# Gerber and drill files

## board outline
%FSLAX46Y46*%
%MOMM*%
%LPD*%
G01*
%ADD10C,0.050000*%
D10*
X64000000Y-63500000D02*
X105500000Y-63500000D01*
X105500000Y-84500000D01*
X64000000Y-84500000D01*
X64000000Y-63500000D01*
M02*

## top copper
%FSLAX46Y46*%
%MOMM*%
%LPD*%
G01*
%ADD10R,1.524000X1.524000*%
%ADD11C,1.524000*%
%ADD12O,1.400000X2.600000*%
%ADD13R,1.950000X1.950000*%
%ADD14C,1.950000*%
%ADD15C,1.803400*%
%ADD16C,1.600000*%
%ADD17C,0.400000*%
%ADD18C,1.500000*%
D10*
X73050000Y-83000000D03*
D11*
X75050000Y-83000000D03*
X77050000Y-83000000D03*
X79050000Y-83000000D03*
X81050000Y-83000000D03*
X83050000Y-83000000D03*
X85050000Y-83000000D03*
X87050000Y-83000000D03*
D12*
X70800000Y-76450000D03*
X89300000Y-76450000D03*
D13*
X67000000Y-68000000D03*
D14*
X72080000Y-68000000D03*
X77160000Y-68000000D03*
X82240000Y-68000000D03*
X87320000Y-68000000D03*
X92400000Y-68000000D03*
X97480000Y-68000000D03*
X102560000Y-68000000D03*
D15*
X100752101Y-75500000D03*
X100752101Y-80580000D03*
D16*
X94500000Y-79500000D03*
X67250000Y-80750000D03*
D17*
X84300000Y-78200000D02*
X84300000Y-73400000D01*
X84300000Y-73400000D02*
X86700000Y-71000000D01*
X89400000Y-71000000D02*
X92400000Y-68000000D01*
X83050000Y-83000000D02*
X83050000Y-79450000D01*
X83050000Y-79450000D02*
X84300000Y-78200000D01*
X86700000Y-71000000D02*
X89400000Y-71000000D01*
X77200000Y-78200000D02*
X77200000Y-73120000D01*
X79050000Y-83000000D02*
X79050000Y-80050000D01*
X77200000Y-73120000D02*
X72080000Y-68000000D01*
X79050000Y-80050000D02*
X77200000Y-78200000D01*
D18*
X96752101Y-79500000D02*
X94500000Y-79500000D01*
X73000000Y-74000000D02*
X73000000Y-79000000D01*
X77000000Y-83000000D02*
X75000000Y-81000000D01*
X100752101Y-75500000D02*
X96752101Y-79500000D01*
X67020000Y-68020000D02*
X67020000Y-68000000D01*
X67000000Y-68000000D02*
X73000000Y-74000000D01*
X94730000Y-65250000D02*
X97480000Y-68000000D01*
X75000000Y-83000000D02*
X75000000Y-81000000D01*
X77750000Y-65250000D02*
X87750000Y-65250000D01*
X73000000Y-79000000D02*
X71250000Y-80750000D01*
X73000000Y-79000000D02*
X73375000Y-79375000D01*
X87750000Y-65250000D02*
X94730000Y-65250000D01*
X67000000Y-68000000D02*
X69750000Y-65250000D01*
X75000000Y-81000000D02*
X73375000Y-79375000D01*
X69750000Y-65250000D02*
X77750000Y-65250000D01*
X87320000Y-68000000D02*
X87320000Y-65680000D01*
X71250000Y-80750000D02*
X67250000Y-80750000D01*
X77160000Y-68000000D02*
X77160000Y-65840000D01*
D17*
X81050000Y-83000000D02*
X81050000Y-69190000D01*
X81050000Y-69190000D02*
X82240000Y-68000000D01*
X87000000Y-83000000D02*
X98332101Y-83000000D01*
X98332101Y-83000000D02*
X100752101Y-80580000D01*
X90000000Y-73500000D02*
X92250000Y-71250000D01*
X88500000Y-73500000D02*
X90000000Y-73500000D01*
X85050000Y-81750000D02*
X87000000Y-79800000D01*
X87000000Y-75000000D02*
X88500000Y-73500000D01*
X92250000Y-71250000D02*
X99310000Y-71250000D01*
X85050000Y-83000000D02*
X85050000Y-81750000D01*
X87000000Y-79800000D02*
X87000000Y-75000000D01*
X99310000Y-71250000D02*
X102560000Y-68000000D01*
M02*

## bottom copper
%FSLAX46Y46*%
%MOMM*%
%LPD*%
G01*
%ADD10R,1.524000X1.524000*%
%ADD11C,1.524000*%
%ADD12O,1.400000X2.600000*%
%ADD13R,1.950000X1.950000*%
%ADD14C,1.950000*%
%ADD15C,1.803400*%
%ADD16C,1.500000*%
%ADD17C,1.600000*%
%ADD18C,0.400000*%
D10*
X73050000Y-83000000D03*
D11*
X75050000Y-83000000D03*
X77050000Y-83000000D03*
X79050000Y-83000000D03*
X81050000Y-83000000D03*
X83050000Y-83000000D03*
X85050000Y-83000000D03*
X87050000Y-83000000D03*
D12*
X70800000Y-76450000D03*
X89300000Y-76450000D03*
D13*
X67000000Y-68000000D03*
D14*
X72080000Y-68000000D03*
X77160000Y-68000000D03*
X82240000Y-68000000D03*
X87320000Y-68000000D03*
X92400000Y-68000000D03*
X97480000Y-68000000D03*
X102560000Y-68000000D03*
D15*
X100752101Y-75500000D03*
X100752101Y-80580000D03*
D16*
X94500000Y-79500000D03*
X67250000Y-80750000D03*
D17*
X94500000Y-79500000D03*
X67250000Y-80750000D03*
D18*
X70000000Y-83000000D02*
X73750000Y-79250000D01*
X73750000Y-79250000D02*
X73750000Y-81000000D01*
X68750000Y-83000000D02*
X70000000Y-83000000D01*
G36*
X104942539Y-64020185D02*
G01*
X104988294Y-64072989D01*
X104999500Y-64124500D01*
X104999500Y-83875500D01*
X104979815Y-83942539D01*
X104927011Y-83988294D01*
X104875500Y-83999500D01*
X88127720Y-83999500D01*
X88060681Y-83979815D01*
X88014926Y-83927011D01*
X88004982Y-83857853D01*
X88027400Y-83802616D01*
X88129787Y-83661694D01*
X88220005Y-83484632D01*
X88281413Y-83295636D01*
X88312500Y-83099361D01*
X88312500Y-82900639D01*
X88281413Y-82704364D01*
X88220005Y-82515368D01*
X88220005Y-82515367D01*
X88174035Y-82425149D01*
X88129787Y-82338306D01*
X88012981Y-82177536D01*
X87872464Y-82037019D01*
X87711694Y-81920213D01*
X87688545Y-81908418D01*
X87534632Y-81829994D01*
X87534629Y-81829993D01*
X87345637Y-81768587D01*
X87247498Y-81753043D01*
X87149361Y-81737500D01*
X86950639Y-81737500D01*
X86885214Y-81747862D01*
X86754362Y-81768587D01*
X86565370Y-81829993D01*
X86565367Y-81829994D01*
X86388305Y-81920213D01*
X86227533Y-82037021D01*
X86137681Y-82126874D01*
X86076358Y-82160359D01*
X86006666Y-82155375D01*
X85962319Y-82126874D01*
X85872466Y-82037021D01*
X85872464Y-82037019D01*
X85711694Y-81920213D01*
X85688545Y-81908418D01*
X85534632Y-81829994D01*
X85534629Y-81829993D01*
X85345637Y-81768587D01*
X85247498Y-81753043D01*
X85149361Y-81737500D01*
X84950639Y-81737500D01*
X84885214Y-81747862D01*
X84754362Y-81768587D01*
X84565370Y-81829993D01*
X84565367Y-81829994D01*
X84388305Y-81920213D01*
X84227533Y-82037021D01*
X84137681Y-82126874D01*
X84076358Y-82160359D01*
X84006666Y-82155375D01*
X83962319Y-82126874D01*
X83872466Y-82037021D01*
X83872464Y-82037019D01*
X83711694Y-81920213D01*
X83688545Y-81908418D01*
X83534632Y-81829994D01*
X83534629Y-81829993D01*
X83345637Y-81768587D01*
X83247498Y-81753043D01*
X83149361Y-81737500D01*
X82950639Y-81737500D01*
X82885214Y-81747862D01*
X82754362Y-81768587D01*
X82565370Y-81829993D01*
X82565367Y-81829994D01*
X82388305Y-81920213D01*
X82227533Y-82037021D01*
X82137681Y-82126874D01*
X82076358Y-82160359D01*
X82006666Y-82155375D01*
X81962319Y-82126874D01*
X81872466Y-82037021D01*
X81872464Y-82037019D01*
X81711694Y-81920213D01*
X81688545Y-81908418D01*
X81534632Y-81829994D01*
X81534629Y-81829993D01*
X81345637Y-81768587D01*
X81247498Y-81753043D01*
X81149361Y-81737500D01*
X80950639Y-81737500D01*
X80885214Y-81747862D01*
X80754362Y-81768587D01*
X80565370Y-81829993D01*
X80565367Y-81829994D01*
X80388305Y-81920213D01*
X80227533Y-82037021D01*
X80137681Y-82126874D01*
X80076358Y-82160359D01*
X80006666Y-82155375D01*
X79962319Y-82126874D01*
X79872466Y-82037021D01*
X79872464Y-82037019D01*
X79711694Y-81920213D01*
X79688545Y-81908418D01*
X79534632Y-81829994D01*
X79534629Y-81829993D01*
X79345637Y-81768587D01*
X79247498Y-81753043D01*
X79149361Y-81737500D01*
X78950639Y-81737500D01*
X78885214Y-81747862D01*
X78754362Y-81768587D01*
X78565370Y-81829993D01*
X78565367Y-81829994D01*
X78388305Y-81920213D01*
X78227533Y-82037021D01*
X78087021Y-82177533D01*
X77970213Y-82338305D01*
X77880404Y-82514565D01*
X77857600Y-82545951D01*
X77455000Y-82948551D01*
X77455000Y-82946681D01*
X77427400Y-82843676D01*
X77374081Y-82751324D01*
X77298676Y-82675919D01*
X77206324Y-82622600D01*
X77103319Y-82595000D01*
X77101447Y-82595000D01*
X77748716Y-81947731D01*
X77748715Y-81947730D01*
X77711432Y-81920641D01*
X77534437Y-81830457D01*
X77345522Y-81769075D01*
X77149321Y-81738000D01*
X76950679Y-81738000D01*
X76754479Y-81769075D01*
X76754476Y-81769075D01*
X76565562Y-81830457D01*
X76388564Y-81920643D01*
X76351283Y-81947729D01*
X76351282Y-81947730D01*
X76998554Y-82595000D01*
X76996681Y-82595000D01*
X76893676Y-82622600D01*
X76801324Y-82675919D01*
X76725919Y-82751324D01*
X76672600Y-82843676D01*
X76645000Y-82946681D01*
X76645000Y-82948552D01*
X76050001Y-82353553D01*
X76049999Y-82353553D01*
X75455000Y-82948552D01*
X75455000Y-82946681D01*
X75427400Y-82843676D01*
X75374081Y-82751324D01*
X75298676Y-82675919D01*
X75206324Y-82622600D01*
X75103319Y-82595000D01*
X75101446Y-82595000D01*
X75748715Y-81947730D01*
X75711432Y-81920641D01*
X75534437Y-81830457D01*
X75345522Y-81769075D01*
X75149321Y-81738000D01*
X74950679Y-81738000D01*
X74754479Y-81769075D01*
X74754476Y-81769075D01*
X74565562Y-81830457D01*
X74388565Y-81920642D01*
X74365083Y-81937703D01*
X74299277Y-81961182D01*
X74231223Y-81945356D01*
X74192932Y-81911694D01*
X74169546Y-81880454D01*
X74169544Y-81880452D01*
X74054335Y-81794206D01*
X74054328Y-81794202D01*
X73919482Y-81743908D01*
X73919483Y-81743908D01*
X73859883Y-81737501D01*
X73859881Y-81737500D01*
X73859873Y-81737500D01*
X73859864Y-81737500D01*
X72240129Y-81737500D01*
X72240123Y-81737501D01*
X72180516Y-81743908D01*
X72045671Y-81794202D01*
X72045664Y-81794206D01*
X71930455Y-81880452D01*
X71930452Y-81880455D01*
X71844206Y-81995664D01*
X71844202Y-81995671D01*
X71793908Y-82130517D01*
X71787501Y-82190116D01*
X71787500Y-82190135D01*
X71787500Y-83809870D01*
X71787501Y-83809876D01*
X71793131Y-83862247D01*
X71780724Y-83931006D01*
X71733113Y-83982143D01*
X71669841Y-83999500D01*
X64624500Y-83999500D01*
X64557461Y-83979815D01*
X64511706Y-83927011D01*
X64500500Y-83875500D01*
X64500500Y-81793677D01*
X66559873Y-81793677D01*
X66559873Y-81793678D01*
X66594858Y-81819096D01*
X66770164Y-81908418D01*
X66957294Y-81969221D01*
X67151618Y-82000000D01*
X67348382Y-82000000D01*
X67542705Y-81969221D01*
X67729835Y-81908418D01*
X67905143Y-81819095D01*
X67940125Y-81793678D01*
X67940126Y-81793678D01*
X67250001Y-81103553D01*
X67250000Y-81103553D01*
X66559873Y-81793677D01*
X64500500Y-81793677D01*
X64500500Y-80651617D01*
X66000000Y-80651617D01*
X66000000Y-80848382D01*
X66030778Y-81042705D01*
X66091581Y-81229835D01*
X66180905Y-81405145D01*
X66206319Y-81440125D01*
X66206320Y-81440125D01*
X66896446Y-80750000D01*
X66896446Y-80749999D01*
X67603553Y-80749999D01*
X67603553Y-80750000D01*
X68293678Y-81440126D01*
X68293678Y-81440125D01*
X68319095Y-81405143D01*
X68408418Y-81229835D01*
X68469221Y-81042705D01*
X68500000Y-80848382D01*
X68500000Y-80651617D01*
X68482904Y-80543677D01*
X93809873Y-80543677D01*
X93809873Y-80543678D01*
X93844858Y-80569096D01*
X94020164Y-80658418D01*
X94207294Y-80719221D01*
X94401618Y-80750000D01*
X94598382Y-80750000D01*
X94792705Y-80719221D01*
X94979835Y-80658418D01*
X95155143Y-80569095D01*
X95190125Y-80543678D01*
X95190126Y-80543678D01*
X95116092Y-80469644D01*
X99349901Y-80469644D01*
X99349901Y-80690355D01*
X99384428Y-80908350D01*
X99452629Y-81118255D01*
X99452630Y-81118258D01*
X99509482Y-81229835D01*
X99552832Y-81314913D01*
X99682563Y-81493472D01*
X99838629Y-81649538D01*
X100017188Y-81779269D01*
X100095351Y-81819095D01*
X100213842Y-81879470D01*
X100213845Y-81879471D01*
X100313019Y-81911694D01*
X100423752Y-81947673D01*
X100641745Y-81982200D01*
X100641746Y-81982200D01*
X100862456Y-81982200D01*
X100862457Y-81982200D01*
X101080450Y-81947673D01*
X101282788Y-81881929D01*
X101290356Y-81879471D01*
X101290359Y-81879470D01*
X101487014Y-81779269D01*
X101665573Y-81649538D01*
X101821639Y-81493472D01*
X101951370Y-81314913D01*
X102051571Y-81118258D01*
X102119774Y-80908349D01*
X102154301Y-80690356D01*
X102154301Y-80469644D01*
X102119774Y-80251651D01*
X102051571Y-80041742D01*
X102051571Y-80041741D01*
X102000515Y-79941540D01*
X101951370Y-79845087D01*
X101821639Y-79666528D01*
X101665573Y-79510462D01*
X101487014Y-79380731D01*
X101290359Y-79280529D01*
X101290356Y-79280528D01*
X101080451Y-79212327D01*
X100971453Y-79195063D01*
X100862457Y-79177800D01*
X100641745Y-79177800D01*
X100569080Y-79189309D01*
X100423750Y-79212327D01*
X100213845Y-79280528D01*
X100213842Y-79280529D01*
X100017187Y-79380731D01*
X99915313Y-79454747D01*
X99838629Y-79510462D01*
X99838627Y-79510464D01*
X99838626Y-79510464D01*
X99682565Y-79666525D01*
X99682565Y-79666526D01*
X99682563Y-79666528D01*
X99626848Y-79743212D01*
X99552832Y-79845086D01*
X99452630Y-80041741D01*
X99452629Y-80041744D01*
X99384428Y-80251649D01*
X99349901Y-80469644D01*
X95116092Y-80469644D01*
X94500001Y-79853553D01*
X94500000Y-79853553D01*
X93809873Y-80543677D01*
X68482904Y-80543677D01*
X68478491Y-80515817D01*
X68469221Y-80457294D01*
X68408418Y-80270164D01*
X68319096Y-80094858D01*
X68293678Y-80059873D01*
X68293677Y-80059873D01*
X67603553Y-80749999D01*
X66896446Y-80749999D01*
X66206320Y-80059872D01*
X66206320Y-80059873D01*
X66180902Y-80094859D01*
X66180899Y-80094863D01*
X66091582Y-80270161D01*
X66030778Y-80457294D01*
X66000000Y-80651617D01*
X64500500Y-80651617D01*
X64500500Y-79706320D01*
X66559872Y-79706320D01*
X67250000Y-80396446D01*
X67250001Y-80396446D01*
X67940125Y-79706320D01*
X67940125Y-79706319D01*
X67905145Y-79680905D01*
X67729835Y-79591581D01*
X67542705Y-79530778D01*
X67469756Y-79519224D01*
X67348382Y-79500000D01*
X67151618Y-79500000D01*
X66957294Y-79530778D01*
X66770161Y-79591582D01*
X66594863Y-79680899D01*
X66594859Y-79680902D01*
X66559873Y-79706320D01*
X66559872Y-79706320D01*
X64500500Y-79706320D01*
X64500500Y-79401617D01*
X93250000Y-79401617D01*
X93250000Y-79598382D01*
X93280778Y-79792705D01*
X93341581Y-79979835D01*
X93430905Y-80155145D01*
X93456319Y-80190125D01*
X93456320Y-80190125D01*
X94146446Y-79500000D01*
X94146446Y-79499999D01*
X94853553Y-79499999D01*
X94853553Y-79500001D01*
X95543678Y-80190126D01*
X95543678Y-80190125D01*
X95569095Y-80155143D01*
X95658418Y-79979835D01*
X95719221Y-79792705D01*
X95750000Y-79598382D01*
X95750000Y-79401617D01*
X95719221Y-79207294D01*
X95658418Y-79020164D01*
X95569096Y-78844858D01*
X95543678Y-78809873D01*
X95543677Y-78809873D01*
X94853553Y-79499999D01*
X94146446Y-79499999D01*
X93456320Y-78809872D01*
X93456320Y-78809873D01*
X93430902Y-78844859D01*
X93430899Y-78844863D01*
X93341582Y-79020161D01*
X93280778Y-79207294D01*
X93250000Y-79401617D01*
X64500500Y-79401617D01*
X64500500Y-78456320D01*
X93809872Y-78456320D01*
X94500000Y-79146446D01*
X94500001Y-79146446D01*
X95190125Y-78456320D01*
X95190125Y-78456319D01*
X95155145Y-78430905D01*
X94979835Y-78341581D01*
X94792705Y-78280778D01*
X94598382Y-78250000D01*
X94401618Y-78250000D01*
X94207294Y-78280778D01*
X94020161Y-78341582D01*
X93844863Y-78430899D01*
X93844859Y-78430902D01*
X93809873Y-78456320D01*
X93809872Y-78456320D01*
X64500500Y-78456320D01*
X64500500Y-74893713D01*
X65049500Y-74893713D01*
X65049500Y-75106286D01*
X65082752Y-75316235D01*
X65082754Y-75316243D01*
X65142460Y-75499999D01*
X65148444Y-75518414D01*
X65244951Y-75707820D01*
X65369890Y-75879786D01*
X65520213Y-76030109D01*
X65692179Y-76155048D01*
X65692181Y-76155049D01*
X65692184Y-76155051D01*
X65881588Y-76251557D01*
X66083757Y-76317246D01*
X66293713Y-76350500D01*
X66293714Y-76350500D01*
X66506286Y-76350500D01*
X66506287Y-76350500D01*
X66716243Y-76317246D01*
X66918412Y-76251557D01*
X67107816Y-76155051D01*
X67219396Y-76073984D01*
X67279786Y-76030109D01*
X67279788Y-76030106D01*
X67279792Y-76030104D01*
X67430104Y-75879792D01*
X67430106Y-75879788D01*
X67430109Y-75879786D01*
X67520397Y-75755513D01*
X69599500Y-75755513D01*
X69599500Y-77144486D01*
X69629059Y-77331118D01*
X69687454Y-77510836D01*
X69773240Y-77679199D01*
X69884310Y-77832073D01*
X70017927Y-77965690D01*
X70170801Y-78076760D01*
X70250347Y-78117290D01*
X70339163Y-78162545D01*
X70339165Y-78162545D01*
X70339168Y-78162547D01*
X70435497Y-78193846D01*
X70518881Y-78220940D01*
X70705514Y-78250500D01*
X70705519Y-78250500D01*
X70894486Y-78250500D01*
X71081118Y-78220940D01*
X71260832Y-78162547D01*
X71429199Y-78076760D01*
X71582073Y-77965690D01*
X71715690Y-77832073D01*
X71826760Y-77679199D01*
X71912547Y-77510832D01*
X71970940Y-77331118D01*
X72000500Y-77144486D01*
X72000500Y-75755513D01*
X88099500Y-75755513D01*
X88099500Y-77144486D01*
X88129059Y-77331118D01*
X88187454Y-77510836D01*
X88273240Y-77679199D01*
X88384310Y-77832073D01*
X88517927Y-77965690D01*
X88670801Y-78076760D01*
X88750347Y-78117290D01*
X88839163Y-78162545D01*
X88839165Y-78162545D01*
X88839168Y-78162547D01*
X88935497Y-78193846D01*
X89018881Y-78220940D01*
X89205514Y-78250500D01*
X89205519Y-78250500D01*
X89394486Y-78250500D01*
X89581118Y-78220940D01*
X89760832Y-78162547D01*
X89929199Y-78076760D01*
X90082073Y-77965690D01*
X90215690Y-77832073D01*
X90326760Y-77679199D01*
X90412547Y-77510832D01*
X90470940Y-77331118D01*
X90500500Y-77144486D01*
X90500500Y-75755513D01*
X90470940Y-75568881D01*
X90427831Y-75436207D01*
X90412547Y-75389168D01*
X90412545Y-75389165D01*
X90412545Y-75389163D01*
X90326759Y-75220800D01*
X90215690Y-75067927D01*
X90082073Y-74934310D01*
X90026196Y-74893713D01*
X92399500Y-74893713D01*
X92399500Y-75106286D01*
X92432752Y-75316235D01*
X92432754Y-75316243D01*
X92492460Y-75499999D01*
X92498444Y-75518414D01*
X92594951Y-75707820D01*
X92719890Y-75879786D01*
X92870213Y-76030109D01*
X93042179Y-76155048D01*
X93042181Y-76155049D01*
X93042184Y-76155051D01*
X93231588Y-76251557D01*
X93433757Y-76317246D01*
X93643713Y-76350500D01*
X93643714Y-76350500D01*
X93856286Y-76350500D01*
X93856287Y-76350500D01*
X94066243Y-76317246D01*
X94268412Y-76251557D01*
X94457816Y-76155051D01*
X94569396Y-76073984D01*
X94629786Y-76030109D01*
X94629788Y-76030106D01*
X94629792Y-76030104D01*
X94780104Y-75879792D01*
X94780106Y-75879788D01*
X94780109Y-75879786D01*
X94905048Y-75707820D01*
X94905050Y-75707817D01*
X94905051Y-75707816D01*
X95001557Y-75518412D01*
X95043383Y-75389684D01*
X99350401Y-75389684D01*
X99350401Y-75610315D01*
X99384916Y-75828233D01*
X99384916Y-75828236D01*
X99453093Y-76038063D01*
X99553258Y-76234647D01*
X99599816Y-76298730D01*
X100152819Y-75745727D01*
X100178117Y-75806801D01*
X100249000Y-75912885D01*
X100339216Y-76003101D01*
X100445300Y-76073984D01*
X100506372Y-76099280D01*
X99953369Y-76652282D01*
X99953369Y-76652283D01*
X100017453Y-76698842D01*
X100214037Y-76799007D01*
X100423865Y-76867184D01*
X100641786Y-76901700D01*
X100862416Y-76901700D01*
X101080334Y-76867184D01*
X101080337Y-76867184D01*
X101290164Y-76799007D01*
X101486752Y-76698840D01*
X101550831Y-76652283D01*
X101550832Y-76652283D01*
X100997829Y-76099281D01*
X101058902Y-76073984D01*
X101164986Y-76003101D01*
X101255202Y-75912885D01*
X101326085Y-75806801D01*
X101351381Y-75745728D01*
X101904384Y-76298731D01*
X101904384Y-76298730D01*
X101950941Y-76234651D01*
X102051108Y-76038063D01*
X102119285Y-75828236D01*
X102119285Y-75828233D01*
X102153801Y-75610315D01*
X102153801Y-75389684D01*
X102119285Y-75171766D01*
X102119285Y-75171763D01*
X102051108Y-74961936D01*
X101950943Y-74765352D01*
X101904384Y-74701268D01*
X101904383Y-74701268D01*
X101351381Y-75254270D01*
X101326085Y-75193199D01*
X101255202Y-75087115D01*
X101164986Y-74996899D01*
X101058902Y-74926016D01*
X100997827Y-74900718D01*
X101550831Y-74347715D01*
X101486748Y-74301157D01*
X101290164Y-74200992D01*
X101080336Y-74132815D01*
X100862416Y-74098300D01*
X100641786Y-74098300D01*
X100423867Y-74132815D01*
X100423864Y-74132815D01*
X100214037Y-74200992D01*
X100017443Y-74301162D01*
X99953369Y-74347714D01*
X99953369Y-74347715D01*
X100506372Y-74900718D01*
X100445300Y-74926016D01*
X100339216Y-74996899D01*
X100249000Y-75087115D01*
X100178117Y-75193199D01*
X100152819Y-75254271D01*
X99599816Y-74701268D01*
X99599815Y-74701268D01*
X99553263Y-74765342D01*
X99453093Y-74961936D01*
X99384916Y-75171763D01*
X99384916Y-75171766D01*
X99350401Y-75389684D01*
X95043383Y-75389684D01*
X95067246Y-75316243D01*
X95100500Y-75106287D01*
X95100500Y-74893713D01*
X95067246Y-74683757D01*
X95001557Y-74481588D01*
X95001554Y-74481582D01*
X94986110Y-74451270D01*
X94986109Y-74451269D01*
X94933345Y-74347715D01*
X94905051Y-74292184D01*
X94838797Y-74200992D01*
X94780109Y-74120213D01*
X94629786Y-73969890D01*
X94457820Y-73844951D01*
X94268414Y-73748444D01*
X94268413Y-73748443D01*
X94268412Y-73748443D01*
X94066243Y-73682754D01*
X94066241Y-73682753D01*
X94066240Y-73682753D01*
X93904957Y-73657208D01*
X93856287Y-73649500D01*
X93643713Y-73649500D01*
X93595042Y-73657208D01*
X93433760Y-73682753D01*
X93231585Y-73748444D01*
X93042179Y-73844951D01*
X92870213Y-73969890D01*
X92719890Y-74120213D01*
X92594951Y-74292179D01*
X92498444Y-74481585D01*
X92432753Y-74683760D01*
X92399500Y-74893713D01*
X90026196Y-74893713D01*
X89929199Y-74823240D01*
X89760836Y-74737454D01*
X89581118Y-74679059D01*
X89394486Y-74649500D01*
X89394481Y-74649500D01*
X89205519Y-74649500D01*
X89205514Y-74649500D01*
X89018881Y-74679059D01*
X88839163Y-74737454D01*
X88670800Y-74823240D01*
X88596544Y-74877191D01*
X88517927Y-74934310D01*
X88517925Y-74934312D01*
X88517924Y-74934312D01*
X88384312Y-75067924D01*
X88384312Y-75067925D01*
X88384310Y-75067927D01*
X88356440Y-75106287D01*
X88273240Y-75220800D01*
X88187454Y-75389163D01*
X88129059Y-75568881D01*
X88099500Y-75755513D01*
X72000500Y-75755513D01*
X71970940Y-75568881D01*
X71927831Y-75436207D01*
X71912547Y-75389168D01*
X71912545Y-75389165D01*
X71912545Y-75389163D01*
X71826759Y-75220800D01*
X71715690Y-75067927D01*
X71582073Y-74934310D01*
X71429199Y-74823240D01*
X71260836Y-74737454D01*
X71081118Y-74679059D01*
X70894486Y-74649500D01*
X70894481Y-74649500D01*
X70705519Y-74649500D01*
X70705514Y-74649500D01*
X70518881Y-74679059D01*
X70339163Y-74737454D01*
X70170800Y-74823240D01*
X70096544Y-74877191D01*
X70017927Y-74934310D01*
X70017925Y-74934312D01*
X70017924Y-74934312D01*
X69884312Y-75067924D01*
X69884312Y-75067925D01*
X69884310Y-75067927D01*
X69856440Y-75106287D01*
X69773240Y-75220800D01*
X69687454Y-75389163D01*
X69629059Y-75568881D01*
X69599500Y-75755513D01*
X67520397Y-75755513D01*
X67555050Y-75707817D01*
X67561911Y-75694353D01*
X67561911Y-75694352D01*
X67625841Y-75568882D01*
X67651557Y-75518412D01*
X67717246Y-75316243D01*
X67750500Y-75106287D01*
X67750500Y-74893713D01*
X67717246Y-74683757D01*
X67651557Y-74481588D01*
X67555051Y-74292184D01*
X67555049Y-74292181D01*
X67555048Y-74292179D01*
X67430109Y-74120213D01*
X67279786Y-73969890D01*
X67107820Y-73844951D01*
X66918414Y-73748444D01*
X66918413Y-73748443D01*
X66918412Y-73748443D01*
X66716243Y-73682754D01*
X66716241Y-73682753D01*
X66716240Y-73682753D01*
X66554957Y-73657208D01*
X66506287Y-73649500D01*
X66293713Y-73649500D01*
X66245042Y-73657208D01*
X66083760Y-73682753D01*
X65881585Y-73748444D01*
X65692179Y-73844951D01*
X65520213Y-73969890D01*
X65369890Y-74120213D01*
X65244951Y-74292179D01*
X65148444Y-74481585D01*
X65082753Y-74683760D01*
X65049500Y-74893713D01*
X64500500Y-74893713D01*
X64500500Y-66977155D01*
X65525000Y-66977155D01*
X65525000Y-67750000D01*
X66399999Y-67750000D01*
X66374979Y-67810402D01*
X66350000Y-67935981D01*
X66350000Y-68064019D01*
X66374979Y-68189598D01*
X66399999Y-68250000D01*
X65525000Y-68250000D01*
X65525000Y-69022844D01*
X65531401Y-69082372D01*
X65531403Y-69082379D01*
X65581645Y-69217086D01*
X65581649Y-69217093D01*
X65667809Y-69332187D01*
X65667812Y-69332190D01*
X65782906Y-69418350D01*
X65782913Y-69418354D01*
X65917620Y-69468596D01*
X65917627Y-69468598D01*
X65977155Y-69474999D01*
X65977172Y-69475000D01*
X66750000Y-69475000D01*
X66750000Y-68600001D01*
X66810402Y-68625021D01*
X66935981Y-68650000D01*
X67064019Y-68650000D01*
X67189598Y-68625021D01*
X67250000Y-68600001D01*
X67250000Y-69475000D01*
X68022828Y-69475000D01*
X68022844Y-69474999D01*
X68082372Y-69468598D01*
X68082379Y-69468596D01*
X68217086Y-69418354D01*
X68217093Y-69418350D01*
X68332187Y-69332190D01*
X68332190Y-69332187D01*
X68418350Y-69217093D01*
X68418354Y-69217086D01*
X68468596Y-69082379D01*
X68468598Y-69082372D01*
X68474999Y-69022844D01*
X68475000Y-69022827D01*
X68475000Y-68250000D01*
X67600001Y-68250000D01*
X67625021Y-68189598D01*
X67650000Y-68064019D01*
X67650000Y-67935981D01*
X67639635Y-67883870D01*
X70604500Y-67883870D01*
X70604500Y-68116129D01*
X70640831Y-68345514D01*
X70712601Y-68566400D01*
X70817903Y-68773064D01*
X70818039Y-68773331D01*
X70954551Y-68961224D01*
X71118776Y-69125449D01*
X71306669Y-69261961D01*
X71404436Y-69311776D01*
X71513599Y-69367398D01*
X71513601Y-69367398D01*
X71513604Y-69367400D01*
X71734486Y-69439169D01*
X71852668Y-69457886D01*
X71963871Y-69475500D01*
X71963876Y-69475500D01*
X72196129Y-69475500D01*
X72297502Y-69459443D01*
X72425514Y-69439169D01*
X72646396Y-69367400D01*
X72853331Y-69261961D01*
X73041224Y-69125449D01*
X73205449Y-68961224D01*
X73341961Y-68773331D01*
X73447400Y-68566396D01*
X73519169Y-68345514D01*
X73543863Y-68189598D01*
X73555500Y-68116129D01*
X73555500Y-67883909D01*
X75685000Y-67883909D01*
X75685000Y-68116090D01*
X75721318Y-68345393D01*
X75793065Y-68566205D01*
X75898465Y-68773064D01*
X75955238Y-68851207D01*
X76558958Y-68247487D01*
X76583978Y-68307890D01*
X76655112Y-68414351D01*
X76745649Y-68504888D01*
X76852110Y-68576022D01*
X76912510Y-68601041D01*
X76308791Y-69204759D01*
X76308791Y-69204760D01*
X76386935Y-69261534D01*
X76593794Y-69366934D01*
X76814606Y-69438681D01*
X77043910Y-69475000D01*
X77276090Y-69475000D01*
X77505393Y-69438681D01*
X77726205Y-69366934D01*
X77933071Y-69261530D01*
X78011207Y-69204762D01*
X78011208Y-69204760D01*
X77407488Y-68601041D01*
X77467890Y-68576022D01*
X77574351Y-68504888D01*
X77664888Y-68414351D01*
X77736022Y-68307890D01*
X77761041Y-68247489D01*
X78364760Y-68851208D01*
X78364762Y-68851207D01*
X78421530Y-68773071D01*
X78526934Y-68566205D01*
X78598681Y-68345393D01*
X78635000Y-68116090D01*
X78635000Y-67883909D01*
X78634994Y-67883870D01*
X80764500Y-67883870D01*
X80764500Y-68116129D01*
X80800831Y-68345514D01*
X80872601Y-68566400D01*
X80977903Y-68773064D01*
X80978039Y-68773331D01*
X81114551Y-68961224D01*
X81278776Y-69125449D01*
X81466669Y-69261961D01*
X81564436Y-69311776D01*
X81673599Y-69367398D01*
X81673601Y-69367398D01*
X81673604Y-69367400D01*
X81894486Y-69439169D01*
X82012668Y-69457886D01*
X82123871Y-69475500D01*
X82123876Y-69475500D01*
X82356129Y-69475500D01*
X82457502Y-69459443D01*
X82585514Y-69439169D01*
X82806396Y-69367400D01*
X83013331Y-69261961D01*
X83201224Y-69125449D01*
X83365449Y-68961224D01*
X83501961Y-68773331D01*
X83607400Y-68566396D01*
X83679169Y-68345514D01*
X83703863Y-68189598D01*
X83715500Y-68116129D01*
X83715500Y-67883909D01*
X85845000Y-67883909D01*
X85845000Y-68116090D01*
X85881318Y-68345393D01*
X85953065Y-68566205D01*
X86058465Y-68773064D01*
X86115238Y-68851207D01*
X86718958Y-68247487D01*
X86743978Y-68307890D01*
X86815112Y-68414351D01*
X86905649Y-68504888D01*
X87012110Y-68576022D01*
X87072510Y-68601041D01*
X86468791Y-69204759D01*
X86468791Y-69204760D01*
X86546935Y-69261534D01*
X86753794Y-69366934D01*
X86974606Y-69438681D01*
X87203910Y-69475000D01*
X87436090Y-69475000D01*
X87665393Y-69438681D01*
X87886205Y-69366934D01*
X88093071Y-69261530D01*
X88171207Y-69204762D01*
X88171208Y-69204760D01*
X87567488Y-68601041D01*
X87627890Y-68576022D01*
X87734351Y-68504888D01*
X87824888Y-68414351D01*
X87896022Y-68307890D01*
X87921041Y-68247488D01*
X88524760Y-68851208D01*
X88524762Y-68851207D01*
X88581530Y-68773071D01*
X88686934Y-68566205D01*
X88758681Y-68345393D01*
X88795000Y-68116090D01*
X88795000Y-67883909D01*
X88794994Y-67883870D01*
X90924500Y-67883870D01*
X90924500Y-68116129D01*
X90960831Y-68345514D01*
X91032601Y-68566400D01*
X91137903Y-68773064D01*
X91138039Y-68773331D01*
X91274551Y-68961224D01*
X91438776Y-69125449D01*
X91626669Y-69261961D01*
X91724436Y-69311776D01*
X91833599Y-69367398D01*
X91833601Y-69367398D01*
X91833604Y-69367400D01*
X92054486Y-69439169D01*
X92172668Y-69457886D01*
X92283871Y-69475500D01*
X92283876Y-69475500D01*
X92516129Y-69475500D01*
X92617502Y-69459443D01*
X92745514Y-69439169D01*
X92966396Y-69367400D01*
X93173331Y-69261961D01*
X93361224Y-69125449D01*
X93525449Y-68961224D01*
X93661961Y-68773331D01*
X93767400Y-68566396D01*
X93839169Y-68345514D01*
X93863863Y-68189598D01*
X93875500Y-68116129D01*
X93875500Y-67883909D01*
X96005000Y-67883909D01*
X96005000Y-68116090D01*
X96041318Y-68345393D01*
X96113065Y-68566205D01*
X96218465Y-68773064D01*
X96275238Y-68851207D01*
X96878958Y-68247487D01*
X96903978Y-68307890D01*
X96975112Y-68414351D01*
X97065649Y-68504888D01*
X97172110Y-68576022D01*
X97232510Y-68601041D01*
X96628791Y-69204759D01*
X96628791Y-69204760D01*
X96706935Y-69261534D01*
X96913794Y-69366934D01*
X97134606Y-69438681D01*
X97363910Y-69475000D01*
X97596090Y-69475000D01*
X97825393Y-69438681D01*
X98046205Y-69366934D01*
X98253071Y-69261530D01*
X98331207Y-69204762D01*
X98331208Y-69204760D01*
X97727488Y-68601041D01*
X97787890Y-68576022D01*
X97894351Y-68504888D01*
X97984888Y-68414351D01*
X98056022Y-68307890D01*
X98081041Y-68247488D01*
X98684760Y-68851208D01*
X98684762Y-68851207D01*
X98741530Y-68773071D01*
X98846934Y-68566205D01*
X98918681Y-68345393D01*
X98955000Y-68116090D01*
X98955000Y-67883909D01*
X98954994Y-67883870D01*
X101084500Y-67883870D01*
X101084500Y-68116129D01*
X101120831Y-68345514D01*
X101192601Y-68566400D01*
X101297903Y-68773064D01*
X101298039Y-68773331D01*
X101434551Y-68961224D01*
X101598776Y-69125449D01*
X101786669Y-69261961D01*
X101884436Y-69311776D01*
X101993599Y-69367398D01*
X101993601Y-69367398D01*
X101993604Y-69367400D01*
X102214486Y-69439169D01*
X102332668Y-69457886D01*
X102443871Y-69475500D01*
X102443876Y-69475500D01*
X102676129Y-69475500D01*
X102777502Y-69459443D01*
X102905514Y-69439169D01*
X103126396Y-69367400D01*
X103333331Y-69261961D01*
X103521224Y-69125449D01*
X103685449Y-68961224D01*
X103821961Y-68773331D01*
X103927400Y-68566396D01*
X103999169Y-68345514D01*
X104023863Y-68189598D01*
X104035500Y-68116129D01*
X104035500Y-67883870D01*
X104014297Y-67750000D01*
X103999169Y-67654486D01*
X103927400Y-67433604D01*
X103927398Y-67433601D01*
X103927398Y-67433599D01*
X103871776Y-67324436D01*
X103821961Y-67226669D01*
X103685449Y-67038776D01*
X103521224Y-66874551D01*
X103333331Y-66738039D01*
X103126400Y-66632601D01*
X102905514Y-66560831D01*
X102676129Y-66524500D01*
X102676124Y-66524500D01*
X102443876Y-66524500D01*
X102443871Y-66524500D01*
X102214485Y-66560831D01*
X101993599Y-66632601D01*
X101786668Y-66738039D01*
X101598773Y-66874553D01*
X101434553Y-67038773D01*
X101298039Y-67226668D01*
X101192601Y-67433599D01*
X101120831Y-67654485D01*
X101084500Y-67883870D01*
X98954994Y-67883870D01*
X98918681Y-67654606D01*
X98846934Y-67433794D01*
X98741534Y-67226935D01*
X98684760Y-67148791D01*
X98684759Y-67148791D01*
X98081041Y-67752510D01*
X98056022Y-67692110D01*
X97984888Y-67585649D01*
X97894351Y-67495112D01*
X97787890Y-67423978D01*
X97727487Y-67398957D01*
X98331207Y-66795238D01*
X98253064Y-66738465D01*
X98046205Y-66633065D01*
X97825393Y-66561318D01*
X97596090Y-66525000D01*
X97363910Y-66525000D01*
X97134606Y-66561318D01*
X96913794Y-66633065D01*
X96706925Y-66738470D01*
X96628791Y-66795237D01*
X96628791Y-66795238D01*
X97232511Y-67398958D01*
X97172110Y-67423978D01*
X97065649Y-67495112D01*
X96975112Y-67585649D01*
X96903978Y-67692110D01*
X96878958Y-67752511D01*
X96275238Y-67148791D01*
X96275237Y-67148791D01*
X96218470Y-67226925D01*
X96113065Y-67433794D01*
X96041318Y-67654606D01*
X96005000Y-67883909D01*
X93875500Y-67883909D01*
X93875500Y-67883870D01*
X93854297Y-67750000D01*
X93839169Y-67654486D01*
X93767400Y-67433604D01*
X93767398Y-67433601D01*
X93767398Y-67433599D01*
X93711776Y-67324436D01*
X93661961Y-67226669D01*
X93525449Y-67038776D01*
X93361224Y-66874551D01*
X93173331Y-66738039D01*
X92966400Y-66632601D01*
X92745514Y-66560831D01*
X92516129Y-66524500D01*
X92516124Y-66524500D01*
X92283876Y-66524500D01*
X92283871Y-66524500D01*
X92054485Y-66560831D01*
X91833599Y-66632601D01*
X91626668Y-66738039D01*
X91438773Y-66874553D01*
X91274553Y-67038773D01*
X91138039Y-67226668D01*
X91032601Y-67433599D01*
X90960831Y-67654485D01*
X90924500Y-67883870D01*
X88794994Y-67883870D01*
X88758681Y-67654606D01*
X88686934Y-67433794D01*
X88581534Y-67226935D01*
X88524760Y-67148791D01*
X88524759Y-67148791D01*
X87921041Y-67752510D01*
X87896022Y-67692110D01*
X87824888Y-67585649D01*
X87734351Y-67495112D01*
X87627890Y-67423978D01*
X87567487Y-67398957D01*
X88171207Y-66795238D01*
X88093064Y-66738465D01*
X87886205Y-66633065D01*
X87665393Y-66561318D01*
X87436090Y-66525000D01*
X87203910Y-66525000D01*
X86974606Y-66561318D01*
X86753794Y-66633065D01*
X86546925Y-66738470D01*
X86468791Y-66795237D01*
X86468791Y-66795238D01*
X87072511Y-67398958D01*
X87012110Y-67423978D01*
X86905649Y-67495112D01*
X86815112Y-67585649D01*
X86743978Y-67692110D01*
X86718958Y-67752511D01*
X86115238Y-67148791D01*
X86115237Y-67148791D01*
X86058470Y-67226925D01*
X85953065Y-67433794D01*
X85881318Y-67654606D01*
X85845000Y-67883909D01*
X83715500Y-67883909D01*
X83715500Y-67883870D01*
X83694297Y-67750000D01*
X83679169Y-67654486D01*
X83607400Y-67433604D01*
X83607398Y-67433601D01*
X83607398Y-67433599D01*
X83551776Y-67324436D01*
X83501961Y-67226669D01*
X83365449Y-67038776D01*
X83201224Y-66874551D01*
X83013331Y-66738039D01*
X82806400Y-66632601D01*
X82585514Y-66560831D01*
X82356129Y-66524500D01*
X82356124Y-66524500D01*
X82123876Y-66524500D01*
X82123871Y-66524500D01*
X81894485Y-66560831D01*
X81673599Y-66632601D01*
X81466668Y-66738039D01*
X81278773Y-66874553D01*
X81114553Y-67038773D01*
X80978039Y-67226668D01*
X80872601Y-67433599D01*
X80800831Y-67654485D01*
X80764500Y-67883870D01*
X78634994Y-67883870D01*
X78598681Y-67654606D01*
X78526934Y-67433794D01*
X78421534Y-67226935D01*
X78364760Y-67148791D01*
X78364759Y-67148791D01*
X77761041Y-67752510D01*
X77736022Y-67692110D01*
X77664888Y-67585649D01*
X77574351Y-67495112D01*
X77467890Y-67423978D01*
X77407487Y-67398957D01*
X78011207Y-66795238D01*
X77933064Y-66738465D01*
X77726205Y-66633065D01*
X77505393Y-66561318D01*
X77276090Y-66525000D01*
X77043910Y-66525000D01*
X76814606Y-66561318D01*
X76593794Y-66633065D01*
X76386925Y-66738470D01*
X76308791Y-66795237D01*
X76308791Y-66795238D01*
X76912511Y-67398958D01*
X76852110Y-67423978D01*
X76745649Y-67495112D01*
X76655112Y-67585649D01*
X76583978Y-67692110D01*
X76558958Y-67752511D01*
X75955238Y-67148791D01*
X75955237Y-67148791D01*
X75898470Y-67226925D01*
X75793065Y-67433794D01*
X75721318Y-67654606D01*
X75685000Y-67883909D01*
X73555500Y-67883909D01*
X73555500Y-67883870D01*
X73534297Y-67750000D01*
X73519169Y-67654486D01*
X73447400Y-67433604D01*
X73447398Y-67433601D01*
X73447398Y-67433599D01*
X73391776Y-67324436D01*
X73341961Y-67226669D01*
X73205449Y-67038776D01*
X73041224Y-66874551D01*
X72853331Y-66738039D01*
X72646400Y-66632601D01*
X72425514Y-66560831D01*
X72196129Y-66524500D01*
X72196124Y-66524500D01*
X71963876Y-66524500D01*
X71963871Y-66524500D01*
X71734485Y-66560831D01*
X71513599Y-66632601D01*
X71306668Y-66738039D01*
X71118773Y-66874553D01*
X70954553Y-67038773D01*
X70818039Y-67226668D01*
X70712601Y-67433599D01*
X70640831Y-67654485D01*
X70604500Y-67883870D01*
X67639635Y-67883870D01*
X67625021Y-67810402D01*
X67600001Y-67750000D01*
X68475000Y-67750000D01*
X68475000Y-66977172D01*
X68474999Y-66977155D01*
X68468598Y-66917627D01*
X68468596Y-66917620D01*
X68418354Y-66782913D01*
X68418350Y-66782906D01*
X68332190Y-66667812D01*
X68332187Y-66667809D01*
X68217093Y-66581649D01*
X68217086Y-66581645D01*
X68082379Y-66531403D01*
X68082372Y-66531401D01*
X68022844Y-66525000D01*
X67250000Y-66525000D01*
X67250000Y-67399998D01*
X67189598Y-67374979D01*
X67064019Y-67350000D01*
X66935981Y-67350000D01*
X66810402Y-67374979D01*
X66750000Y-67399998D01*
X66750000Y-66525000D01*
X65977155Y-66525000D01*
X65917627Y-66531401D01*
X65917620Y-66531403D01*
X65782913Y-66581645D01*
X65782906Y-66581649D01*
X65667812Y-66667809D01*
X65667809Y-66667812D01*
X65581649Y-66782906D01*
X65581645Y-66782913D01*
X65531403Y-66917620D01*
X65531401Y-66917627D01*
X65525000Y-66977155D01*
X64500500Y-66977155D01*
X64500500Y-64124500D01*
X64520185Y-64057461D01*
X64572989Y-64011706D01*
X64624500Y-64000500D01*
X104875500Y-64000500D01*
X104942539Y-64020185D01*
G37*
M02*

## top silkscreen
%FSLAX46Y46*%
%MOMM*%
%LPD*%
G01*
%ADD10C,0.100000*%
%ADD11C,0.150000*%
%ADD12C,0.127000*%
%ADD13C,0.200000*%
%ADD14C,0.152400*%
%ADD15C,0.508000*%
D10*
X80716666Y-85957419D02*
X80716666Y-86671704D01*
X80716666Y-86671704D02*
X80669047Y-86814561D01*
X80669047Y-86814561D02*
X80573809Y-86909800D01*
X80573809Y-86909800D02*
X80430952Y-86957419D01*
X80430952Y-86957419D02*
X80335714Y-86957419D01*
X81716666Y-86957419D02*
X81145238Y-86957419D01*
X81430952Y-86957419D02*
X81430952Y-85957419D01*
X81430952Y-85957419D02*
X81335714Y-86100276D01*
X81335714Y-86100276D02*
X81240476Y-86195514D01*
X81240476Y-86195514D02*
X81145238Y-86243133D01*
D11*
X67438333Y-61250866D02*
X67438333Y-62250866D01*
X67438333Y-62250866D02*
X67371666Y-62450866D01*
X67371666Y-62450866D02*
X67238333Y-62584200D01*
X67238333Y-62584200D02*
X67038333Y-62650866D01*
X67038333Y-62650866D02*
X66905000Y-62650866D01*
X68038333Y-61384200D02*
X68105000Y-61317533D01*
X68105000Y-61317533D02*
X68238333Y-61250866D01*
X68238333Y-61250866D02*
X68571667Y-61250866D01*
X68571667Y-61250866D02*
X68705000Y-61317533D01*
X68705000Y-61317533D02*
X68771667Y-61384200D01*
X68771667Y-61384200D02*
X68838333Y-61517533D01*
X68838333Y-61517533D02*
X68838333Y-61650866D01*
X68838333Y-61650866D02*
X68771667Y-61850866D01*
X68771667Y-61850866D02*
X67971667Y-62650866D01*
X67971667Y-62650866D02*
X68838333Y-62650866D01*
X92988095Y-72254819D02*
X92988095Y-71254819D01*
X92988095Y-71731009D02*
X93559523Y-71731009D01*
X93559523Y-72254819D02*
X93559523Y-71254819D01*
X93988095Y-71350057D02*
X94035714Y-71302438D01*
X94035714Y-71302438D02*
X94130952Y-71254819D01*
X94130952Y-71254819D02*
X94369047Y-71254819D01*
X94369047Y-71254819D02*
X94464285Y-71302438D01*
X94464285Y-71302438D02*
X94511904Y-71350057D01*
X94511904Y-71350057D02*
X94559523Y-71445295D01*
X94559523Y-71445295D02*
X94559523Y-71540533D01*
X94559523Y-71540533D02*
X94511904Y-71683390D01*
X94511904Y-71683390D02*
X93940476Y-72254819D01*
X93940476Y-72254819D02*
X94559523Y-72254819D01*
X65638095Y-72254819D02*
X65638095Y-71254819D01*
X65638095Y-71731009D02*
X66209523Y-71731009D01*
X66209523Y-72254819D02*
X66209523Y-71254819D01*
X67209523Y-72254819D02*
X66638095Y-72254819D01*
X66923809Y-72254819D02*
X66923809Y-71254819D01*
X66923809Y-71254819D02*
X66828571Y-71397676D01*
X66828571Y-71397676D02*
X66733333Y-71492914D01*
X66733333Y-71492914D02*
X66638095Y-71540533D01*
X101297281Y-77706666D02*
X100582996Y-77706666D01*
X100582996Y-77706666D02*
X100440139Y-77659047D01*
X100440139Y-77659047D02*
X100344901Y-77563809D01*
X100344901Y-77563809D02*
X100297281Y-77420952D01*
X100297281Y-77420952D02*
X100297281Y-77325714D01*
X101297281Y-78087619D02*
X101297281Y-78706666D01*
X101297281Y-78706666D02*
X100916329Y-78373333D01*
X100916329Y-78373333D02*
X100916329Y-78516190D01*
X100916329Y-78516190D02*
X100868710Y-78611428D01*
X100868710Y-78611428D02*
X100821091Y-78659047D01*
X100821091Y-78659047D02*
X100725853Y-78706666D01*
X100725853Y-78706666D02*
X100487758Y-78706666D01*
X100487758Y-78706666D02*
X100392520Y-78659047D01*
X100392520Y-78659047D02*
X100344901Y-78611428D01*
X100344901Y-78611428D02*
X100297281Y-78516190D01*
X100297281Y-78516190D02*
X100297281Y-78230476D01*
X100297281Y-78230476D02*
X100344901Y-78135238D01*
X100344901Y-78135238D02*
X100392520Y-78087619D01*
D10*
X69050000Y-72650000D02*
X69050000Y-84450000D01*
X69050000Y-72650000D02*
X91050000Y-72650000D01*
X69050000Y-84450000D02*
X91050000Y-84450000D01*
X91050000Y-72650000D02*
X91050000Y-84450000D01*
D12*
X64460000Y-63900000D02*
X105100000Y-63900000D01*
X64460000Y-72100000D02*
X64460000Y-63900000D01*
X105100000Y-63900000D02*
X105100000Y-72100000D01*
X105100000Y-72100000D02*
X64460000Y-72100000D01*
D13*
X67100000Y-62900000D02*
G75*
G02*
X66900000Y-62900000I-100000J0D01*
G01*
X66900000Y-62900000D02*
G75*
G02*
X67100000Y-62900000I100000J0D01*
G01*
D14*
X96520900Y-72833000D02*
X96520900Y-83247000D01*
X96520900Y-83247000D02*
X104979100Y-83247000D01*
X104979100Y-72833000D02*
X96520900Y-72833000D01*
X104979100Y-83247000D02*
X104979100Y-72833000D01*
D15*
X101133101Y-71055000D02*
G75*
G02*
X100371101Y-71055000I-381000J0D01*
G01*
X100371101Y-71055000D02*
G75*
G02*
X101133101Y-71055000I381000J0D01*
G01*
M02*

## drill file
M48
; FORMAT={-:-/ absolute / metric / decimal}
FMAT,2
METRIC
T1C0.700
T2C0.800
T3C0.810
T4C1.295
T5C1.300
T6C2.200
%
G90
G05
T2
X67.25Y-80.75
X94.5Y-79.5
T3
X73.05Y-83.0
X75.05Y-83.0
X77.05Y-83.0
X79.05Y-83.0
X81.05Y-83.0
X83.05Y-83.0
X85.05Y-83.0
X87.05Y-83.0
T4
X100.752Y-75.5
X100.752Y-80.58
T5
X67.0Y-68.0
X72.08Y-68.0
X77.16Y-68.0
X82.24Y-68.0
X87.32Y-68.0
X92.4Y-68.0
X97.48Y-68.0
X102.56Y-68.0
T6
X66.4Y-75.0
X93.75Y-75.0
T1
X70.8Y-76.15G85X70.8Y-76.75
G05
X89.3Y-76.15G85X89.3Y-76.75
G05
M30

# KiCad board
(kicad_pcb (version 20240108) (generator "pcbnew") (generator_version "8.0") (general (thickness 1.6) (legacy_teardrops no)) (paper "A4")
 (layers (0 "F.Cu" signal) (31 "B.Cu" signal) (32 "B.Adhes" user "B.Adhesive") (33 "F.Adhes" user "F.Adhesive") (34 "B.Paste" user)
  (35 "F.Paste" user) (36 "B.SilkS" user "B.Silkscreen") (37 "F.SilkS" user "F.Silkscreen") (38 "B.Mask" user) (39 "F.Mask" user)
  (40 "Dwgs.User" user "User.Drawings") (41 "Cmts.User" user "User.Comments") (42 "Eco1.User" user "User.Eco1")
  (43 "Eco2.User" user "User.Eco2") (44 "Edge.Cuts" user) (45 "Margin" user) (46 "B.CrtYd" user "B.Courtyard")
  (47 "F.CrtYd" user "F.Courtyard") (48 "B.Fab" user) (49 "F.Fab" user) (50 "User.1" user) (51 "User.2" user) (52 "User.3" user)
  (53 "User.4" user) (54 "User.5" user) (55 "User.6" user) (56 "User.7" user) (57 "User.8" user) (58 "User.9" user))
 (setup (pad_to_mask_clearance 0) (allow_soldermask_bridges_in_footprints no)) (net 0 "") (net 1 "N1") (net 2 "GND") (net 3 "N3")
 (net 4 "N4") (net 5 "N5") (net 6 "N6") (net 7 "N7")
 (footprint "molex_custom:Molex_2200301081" (layer "F.Cu") (at 81.05 87)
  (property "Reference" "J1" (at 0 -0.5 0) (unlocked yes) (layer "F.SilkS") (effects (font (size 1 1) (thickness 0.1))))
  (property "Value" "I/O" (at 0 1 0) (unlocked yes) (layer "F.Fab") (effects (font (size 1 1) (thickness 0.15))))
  (fp_line (start -12 -14.35) (end -12 -2.55) (stroke (width 0.1) (type default)) (layer "F.SilkS"))
  (fp_line (start -12 -14.35) (end 10 -14.35) (stroke (width 0.1) (type default)) (layer "F.SilkS"))
  (fp_line (start -12 -2.55) (end 10 -2.55) (stroke (width 0.1) (type default)) (layer "F.SilkS"))
  (fp_line (start 10 -14.35) (end 10 -2.55) (stroke (width 0.1) (type default)) (layer "F.SilkS"))
  (pad "1" thru_hole rect (at -8 -4 90) (size 1.524 1.524) (drill 0.81) (layers "*.Cu" "*.Mask") (remove_unused_layers no) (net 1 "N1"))
  (pad "2" thru_hole circle (at -6 -4 90) (size 1.524 1.524) (drill 0.81) (layers "*.Cu" "*.Mask") (remove_unused_layers no) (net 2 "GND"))
  (pad "3" thru_hole circle (at -4 -4 90) (size 1.524 1.524) (drill 0.81) (layers "*.Cu" "*.Mask") (remove_unused_layers no) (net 2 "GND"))
  (pad "4" thru_hole circle (at -2 -4 90) (size 1.524 1.524) (drill 0.81) (layers "*.Cu" "*.Mask") (remove_unused_layers no) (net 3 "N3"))
  (pad "5" thru_hole circle (at 0 -4 90) (size 1.524 1.524) (drill 0.81) (layers "*.Cu" "*.Mask") (remove_unused_layers no) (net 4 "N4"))
  (pad "6" thru_hole circle (at 2 -4 90) (size 1.524 1.524) (drill 0.81) (layers "*.Cu" "*.Mask") (remove_unused_layers no) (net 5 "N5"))
  (pad "7" thru_hole circle (at 4 -4 90) (size 1.524 1.524) (drill 0.81) (layers "*.Cu" "*.Mask") (remove_unused_layers no) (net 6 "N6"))
  (pad "8" thru_hole circle (at 6 -4 90) (size 1.524 1.524) (drill 0.81) (layers "*.Cu" "*.Mask") (remove_unused_layers no) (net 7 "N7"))
  (pad "9" thru_hole oval (at -10.25 -10.55 270) (size 2.6 1.4) (drill oval 1.3 0.7) (layers "*.Cu" "*.Mask") (remove_unused_layers no))
  (pad "9" thru_hole oval (at 8.25 -10.55 270) (size 2.6 1.4) (drill oval 1.3 0.7) (layers "*.Cu" "*.Mask") (remove_unused_layers no)))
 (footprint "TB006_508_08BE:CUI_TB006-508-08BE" (layer "F.Cu") (at 67 68)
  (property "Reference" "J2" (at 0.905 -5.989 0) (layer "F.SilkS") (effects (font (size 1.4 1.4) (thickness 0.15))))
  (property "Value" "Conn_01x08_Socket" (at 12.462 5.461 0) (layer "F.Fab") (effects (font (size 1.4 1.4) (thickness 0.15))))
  (fp_line (start -2.54 -4.1) (end 38.1 -4.1) (stroke (width 0.127) (type solid)) (layer "F.SilkS"))
  (fp_line (start -2.54 4.1) (end -2.54 -4.1) (stroke (width 0.127) (type solid)) (layer "F.SilkS"))
  (fp_line (start 38.1 -4.1) (end 38.1 4.1) (stroke (width 0.127) (type solid)) (layer "F.SilkS"))
  (fp_line (start 38.1 4.1) (end -2.54 4.1) (stroke (width 0.127) (type solid)) (layer "F.SilkS"))
  (fp_circle (center 0 -5.1) (end 0.1 -5.1) (stroke (width 0.2) (type solid)) (fill none) (layer "F.SilkS"))
  (pad "1" thru_hole rect (at 0 0) (size 1.95 1.95) (drill 1.3) (layers "*.Cu" "*.Mask") (remove_unused_layers no) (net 2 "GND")
   (solder_mask_margin 0.102))
  (pad "2" thru_hole circle (at 5.08 0) (size 1.95 1.95) (drill 1.3) (layers "*.Cu" "*.Mask") (remove_unused_layers no) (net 3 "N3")
   (solder_mask_margin 0.102))
  (pad "3" thru_hole circle (at 10.16 0) (size 1.95 1.95) (drill 1.3) (layers "*.Cu" "*.Mask") (remove_unused_layers no) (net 2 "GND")
   (solder_mask_margin 0.102))
  (pad "4" thru_hole circle (at 15.24 0) (size 1.95 1.95) (drill 1.3) (layers "*.Cu" "*.Mask") (remove_unused_layers no) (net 4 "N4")
   (solder_mask_margin 0.102))
  (pad "5" thru_hole circle (at 20.32 0) (size 1.95 1.95) (drill 1.3) (layers "*.Cu" "*.Mask") (remove_unused_layers no) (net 2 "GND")
   (solder_mask_margin 0.102))
  (pad "6" thru_hole circle (at 25.4 0) (size 1.95 1.95) (drill 1.3) (layers "*.Cu" "*.Mask") (remove_unused_layers no) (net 5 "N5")
   (solder_mask_margin 0.102))
  (pad "7" thru_hole circle (at 30.48 0) (size 1.95 1.95) (drill 1.3) (layers "*.Cu" "*.Mask") (remove_unused_layers no) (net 2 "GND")
   (solder_mask_margin 0.102))
  (pad "8" thru_hole circle (at 35.56 0) (size 1.95 1.95) (drill 1.3) (layers "*.Cu" "*.Mask") (remove_unused_layers no) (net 6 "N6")
   (solder_mask_margin 0.102)))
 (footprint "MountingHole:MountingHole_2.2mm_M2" (layer "F.Cu") (at 93.75 75)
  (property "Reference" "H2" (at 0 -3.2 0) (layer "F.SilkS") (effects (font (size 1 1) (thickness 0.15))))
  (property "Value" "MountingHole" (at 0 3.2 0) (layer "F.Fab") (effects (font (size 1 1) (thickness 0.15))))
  (pad "" np_thru_hole circle (at 0 0) (size 2.2 2.2) (drill 2.2) (layers "*.Cu" "*.Mask")))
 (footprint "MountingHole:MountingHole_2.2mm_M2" (layer "F.Cu") (at 66.4 75)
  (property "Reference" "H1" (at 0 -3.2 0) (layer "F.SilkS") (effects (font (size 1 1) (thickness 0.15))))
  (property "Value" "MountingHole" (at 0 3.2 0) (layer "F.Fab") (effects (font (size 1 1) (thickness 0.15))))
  (pad "" np_thru_hole circle (at 0 0) (size 2.2 2.2) (drill 2.2) (layers "*.Cu" "*.Mask")))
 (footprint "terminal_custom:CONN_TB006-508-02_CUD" (layer "F.Cu") (at 100.752101 75.5 -90)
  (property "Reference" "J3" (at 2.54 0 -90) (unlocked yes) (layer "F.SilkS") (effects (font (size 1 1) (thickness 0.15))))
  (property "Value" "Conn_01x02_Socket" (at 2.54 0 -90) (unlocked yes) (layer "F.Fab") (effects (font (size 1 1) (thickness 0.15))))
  (fp_line (start -2.667 4.231201) (end 7.747 4.231201) (stroke (width 0.1524) (type solid)) (layer "F.SilkS"))
  (fp_line (start 7.747 4.231201) (end 7.747 -4.226999) (stroke (width 0.1524) (type solid)) (layer "F.SilkS"))
  (fp_line (start -2.667 -4.226999) (end -2.667 4.231201) (stroke (width 0.1524) (type solid)) (layer "F.SilkS"))
  (fp_line (start 7.747 -4.226999) (end -2.667 -4.226999) (stroke (width 0.1524) (type solid)) (layer "F.SilkS"))
  (fp_circle (center -4.445 0) (end -4.064 0) (stroke (width 0.508) (type solid)) (fill none) (layer "F.SilkS"))
  (pad "1" thru_hole circle (at 0 0 270) (size 1.8034 1.8034) (drill 1.2954) (layers "*.Cu" "*.Mask") (remove_unused_layers no)
   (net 2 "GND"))
  (pad "2" thru_hole circle (at 5.08 0 270) (size 1.8034 1.8034) (drill 1.2954) (layers "*.Cu" "*.Mask") (remove_unused_layers no)
   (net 7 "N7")))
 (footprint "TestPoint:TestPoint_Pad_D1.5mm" (layer "B.Cu") (at 94.5 79.5 180)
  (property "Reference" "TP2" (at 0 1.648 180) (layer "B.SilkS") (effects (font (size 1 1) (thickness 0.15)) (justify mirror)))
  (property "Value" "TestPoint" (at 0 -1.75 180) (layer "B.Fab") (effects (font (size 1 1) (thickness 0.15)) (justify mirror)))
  (pad "1" smd circle (at 0 0 180) (size 1.5 1.5) (layers "B.Cu" "B.Mask") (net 2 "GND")))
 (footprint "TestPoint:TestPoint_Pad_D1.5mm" (layer "B.Cu") (at 67.25 80.75 180)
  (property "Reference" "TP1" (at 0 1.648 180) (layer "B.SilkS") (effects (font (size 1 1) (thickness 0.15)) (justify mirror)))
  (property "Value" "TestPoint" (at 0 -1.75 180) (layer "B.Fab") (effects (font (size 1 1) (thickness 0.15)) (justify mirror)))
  (pad "1" smd circle (at 0 0 180) (size 1.5 1.5) (layers "B.Cu" "B.Mask") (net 2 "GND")))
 (gr_rect (start 64 63.5) (end 105.5 84.5) (stroke (width 0.05) (type default)) (fill none) (layer "Edge.Cuts"))
 (segment (start 84.3 78.2) (end 84.3 73.4) (width 0.4) (layer "F.Cu") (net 5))
 (segment (start 84.3 73.4) (end 86.7 71) (width 0.4) (layer "F.Cu") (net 5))
 (segment (start 89.4 71) (end 92.4 68) (width 0.4) (layer "F.Cu") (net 5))
 (segment (start 83.05 83) (end 83.05 79.45) (width 0.4) (layer "F.Cu") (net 5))
 (segment (start 83.05 79.45) (end 84.3 78.2) (width 0.4) (layer "F.Cu") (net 5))
 (segment (start 86.7 71) (end 89.4 71) (width 0.4) (layer "F.Cu") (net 5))
 (segment (start 77.2 78.2) (end 77.2 73.12) (width 0.4) (layer "F.Cu") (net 3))
 (segment (start 79.05 83) (end 79.05 80.05) (width 0.4) (layer "F.Cu") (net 3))
 (segment (start 77.2 73.12) (end 72.08 68) (width 0.4) (layer "F.Cu") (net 3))
 (segment (start 79.05 80.05) (end 77.2 78.2) (width 0.4) (layer "F.Cu") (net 3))
 (segment (start 96.752101 79.5) (end 94.5 79.5) (width 1.5) (layer "F.Cu") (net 2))
 (segment (start 73 74) (end 73 79) (width 1.5) (layer "F.Cu") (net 2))
 (segment (start 77 83) (end 75 81) (width 1.5) (layer "F.Cu") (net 2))
 (segment (start 100.752101 75.5) (end 96.752101 79.5) (width 1.5) (layer "F.Cu") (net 2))
 (segment (start 67.02 68.02) (end 67.02 68) (width 1.5) (layer "F.Cu") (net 2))
 (segment (start 67 68) (end 73 74) (width 1.5) (layer "F.Cu") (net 2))
 (segment (start 94.73 65.25) (end 97.48 68) (width 1.5) (layer "F.Cu") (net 2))
 (segment (start 75 83) (end 75 81) (width 1.5) (layer "F.Cu") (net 2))
 (segment (start 77.75 65.25) (end 87.75 65.25) (width 1.5) (layer "F.Cu") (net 2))
 (segment (start 73 79) (end 71.25 80.75) (width 1.5) (layer "F.Cu") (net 2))
 (segment (start 73 79) (end 73.375 79.375) (width 1.5) (layer "F.Cu") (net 2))
 (segment (start 87.75 65.25) (end 94.73 65.25) (width 1.5) (layer "F.Cu") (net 2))
 (segment (start 67 68) (end 69.75 65.25) (width 1.5) (layer "F.Cu") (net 2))
 (segment (start 75 81) (end 73.375 79.375) (width 1.5) (layer "F.Cu") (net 2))
 (segment (start 69.75 65.25) (end 77.75 65.25) (width 1.5) (layer "F.Cu") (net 2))
 (segment (start 87.32 68) (end 87.32 65.68) (width 1.5) (layer "F.Cu") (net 2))
 (segment (start 71.25 80.75) (end 67.25 80.75) (width 1.5) (layer "F.Cu") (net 2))
 (segment (start 77.16 68) (end 77.16 65.84) (width 1.5) (layer "F.Cu") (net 2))
 (via (at 94.5 79.5) (size 1.6) (drill 0.8) (layers "F.Cu" "B.Cu") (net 2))
 (via (at 67.25 80.75) (size 1.6) (drill 0.8) (layers "F.Cu" "B.Cu") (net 2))
 (segment (start 70 83) (end 73.75 79.25) (width 0.4) (layer "B.Cu") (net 2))
 (segment (start 73.75 79.25) (end 73.75 81) (width 0.4) (layer "B.Cu") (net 2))
 (segment (start 68.75 83) (end 70 83) (width 0.4) (layer "B.Cu") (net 2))
 (segment (start 81.05 83) (end 81.05 69.19) (width 0.4) (layer "F.Cu") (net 4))
 (segment (start 81.05 69.19) (end 82.24 68) (width 0.4) (layer "F.Cu") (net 4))
 (segment (start 87 83) (end 98.332101 83) (width 0.4) (layer "F.Cu") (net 7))
 (segment (start 98.332101 83) (end 100.752101 80.58) (width 0.4) (layer "F.Cu") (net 7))
 (segment (start 90 73.5) (end 92.25 71.25) (width 0.4) (layer "F.Cu") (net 6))
 (segment (start 88.5 73.5) (end 90 73.5) (width 0.4) (layer "F.Cu") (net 6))
 (segment (start 85.05 81.75) (end 87 79.8) (width 0.4) (layer "F.Cu") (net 6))
 (segment (start 87 75) (end 88.5 73.5) (width 0.4) (layer "F.Cu") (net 6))
 (segment (start 92.25 71.25) (end 99.31 71.25) (width 0.4) (layer "F.Cu") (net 6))
 (segment (start 85.05 83) (end 85.05 81.75) (width 0.4) (layer "F.Cu") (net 6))
 (segment (start 87 79.8) (end 87 75) (width 0.4) (layer "F.Cu") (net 6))
 (segment (start 99.31 71.25) (end 102.56 68) (width 0.4) (layer "F.Cu") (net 6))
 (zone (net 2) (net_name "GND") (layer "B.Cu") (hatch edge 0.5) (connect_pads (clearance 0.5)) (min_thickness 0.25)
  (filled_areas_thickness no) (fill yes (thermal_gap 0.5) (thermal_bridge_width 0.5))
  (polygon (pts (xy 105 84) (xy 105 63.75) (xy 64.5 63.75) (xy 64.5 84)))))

